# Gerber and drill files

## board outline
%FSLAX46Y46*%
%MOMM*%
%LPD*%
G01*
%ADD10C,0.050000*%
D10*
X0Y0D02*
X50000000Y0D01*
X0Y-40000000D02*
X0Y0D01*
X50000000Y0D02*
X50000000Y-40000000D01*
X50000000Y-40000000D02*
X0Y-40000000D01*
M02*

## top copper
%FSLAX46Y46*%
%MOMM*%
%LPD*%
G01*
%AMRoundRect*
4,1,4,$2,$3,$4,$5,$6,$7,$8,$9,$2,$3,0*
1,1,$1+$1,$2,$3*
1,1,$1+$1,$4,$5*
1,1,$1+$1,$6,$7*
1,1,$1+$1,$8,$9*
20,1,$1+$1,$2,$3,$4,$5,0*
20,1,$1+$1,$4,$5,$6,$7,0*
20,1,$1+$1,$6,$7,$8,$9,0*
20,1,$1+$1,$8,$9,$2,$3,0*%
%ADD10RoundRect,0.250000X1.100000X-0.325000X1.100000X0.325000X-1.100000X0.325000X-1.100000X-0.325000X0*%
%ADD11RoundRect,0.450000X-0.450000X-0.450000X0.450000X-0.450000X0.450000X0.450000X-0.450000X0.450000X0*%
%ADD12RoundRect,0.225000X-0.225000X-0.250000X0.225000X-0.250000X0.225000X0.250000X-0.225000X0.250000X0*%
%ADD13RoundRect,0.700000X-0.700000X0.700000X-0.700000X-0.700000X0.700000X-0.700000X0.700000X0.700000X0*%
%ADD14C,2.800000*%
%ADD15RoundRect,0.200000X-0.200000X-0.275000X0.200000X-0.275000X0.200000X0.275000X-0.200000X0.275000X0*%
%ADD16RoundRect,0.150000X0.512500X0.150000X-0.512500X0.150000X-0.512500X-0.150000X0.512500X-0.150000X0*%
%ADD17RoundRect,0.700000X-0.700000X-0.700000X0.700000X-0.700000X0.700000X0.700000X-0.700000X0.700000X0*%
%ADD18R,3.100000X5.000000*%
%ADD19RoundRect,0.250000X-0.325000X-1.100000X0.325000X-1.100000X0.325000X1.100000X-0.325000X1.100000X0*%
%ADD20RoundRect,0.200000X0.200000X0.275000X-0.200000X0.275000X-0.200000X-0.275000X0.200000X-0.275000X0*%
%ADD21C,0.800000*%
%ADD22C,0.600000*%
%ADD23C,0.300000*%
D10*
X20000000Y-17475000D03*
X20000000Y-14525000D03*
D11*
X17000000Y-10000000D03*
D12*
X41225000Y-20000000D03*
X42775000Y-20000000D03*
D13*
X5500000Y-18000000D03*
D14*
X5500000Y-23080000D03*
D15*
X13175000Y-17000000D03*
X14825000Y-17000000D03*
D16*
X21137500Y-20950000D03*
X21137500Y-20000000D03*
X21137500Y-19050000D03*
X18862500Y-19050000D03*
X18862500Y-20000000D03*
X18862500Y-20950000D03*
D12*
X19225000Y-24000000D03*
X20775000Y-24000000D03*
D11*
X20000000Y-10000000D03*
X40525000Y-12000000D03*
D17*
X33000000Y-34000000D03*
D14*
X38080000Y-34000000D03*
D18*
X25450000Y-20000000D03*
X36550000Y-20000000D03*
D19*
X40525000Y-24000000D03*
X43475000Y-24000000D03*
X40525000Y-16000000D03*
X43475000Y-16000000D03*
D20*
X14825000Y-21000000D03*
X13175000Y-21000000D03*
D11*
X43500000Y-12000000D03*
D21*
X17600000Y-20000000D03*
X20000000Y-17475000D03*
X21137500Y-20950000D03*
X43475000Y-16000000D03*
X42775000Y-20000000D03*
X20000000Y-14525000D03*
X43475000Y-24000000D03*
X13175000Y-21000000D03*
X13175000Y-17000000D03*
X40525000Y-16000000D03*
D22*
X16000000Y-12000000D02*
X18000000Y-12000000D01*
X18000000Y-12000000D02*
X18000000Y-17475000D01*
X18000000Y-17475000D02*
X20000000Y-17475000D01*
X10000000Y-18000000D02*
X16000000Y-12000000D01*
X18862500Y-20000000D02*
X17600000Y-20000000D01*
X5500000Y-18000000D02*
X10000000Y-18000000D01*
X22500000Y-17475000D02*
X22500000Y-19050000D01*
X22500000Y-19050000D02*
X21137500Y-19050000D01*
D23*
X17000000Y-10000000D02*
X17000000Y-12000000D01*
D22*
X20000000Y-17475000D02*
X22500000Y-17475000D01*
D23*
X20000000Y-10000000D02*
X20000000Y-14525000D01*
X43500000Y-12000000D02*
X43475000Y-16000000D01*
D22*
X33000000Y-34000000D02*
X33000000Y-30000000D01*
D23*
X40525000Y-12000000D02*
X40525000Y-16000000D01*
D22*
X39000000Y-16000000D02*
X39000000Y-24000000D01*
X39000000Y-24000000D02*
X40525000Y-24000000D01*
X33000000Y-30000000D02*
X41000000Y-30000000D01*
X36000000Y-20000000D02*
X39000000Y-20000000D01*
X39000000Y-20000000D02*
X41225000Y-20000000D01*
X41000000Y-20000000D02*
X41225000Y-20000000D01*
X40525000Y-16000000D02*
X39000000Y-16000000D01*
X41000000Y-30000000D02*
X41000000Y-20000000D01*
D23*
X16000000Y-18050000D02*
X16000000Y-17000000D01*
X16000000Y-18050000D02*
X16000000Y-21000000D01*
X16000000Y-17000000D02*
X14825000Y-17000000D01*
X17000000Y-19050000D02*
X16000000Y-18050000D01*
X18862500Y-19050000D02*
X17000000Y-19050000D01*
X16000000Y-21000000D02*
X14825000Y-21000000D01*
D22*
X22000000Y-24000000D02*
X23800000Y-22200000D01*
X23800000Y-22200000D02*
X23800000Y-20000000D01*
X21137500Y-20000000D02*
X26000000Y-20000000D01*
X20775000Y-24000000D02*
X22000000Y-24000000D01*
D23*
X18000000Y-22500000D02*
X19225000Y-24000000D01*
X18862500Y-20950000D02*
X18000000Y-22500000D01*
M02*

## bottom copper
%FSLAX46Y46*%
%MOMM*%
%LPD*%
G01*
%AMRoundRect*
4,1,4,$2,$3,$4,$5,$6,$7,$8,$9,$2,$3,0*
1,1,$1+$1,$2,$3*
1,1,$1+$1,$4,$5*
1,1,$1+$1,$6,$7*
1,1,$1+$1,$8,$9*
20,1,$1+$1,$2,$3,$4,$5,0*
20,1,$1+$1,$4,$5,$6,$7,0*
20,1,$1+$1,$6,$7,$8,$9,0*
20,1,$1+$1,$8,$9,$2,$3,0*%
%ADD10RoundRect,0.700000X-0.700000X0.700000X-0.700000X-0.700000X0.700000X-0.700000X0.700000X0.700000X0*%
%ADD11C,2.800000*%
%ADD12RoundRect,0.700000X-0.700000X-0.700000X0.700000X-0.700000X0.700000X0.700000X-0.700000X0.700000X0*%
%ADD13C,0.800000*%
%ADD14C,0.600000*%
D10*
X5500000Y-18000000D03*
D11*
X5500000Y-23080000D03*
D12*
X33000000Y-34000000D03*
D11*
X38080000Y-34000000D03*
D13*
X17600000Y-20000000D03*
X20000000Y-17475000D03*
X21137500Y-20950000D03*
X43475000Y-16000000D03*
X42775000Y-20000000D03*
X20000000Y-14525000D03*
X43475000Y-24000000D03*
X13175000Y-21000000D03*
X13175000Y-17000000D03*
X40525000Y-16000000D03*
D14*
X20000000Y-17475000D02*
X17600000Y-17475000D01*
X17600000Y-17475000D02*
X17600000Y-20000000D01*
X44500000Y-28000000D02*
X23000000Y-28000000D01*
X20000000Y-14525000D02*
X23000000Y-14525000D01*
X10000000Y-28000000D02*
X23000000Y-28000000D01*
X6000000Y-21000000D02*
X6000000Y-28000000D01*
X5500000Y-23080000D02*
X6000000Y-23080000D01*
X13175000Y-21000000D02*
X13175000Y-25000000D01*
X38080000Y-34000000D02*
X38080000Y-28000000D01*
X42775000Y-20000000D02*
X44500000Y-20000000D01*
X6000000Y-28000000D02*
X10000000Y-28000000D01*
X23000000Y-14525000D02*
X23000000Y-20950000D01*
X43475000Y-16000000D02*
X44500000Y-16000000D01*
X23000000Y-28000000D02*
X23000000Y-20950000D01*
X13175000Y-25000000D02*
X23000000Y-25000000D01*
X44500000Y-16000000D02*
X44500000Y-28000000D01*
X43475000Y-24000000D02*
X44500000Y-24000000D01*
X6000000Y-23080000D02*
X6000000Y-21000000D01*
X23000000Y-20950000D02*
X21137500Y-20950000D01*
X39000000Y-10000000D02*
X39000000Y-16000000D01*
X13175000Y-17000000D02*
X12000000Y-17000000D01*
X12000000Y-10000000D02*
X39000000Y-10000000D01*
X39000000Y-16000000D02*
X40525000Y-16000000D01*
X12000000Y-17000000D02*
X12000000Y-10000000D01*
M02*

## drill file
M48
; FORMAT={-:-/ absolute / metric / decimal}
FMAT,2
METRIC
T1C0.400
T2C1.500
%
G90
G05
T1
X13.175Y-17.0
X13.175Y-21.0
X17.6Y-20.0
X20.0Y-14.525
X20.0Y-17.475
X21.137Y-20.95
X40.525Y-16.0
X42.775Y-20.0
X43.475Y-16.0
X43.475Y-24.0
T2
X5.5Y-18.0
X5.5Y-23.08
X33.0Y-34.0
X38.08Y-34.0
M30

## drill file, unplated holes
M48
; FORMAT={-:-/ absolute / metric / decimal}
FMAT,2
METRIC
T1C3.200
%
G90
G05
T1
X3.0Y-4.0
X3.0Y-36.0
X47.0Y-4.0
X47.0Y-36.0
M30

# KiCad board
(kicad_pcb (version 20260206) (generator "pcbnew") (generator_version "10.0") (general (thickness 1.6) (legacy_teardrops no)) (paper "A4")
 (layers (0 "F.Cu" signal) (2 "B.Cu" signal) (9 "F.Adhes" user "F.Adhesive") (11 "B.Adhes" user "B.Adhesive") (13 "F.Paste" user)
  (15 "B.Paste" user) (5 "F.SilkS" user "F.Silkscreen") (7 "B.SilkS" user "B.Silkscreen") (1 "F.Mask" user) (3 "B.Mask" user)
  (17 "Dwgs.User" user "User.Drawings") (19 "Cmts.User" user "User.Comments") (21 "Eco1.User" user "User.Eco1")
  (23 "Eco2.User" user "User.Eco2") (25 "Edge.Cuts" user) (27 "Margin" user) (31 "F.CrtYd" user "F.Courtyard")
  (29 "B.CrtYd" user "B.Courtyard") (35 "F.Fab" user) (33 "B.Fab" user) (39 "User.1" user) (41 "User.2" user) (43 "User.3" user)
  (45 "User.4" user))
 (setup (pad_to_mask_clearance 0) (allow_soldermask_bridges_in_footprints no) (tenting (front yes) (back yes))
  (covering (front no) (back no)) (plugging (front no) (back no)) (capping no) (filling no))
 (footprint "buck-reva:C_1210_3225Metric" (layer "F.Cu") (at 20 16 90)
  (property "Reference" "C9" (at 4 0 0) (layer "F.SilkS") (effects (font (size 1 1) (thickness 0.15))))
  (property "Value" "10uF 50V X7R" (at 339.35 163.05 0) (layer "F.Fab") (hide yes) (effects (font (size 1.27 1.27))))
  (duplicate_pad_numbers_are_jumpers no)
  (pad "1" smd roundrect (at -1.475 0 90) (size 1.15 2.7) (layers "F.Cu" "F.Mask" "F.Paste") (roundrect_rratio 0.217391) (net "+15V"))
  (pad "2" smd roundrect (at 1.475 0 90) (size 1.15 2.7) (layers "F.Cu" "F.Mask" "F.Paste") (roundrect_rratio 0.217391) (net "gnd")))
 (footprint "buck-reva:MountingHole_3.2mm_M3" (layer "F.Cu") (at 3 36)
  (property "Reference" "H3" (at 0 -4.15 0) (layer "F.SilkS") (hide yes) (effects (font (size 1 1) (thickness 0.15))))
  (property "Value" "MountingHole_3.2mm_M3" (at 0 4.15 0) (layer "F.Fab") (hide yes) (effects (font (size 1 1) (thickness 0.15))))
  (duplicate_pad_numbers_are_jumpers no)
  (pad "" np_thru_hole circle (at 0 0) (size 3.2 3.2) (drill 3.2) (layers "*.Cu" "*.Mask")))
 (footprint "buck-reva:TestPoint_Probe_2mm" (layer "F.Cu") (at 17 10)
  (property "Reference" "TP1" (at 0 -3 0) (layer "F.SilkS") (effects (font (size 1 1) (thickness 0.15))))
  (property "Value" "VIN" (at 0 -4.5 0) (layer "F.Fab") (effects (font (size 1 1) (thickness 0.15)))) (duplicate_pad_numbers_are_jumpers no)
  (pad "1" smd roundrect (at 0 0) (size 1.8 1.8) (layers "F.Cu" "F.Mask") (roundrect_rratio 0.25) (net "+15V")))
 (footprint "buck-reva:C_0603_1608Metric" (layer "F.Cu") (at 42 20)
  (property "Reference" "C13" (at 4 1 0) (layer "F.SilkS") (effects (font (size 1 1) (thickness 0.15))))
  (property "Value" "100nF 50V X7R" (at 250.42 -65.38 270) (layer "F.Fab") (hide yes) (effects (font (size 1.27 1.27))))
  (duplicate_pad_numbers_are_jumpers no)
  (pad "1" smd roundrect (at -0.775 0) (size 0.9 0.95) (layers "F.Cu" "F.Mask" "F.Paste") (roundrect_rratio 0.25) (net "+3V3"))
  (pad "2" smd roundrect (at 0.775 0) (size 0.9 0.95) (layers "F.Cu" "F.Mask" "F.Paste") (roundrect_rratio 0.25) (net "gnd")))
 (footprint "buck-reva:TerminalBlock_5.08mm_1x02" (layer "F.Cu") (at 5.5 18 -90)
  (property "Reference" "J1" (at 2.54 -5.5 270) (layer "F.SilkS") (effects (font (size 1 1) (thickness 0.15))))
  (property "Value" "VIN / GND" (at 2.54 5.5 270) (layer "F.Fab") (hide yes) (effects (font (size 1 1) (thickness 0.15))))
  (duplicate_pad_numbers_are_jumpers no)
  (pad "1" thru_hole roundrect (at 0 0 270) (size 2.8 2.8) (drill 1.5) (layers "*.Cu" "*.Mask") (remove_unused_layers no)
   (roundrect_rratio 0.25) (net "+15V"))
  (pad "2" thru_hole circle (at 5.08 0 270) (size 2.8 2.8) (drill 1.5) (layers "*.Cu" "*.Mask") (remove_unused_layers no) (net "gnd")))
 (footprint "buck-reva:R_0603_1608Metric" (layer "F.Cu") (at 14 17)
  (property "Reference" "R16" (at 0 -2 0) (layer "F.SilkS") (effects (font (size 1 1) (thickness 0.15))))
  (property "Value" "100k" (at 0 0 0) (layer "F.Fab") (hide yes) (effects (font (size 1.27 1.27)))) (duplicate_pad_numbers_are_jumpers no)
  (pad "1" smd roundrect (at -0.825 0) (size 0.8 0.95) (layers "F.Cu" "F.Mask" "F.Paste") (roundrect_rratio 0.25) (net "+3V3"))
  (pad "2" smd roundrect (at 0.825 0) (size 0.8 0.95) (layers "F.Cu" "F.Mask" "F.Paste") (roundrect_rratio 0.25) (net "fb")))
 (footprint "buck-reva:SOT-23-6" (layer "F.Cu") (at 20 20 180)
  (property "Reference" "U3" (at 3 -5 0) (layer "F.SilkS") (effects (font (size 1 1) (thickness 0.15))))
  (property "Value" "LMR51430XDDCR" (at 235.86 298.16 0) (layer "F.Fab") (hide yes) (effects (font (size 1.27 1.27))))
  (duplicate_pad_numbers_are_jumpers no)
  (pad "1" smd roundrect (at -1.1375 -0.95 180) (size 1.325 0.6) (layers "F.Cu" "F.Mask" "F.Paste") (roundrect_rratio 0.25) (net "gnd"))
  (pad "2" smd roundrect (at -1.1375 0 180) (size 1.325 0.6) (layers "F.Cu" "F.Mask" "F.Paste") (roundrect_rratio 0.25) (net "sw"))
  (pad "3" smd roundrect (at -1.1375 0.95 180) (size 1.325 0.6) (layers "F.Cu" "F.Mask" "F.Paste") (roundrect_rratio 0.25) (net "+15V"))
  (pad "4" smd roundrect (at 1.1375 0.95 180) (size 1.325 0.6) (layers "F.Cu" "F.Mask" "F.Paste") (roundrect_rratio 0.25) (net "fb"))
  (pad "5" smd roundrect (at 1.1375 0 180) (size 1.325 0.6) (layers "F.Cu" "F.Mask" "F.Paste") (roundrect_rratio 0.25) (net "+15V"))
  (pad "6" smd roundrect (at 1.1375 -0.95 180) (size 1.325 0.6) (layers "F.Cu" "F.Mask" "F.Paste") (roundrect_rratio 0.25) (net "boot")))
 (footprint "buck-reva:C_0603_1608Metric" (layer "F.Cu") (at 20 24)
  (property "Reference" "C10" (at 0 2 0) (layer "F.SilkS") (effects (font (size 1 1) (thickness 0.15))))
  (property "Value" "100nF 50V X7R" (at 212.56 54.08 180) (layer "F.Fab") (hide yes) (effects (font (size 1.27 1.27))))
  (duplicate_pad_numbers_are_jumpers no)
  (pad "1" smd roundrect (at -0.775 0) (size 0.9 0.95) (layers "F.Cu" "F.Mask" "F.Paste") (roundrect_rratio 0.25) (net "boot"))
  (pad "2" smd roundrect (at 0.775 0) (size 0.9 0.95) (layers "F.Cu" "F.Mask" "F.Paste") (roundrect_rratio 0.25) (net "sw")))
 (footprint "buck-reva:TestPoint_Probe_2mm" (layer "F.Cu") (at 20 10)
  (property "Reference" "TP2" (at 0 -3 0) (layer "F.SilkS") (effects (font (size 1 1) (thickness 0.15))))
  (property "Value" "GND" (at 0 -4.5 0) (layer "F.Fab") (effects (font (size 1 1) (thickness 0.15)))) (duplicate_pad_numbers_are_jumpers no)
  (pad "1" smd roundrect (at 0 0) (size 1.8 1.8) (layers "F.Cu" "F.Mask") (roundrect_rratio 0.25) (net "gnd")))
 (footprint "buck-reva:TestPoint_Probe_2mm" (layer "F.Cu") (at 40.525 12)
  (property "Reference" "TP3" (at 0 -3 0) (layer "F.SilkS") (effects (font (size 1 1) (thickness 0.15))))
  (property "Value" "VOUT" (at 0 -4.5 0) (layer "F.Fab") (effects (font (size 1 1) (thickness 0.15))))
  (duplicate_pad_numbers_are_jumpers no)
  (pad "1" smd roundrect (at 0 0) (size 1.8 1.8) (layers "F.Cu" "F.Mask") (roundrect_rratio 0.25) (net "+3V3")))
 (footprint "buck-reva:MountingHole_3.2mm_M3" (layer "F.Cu") (at 47 4)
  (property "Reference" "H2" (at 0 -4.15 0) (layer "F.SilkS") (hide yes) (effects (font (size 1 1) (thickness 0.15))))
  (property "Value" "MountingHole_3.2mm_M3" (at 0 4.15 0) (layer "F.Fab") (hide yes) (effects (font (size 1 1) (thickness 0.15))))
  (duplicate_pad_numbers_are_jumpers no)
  (pad "" np_thru_hole circle (at 0 0) (size 3.2 3.2) (drill 3.2) (layers "*.Cu" "*.Mask")))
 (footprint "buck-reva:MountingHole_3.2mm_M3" (layer "F.Cu") (at 3 4)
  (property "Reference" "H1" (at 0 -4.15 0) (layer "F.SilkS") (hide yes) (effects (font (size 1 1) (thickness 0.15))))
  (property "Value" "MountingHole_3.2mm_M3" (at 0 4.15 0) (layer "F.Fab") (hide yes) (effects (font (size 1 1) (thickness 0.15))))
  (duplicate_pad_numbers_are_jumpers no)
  (pad "" np_thru_hole circle (at 0 0) (size 3.2 3.2) (drill 3.2) (layers "*.Cu" "*.Mask")))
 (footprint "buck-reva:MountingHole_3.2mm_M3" (layer "F.Cu") (at 47 36)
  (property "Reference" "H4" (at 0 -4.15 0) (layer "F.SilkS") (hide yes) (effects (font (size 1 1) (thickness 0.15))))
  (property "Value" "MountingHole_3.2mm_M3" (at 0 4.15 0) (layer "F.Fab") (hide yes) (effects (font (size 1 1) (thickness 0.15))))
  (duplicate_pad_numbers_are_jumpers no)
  (pad "" np_thru_hole circle (at 0 0) (size 3.2 3.2) (drill 3.2) (layers "*.Cu" "*.Mask")))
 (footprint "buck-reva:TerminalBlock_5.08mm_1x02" (layer "F.Cu") (at 33 34)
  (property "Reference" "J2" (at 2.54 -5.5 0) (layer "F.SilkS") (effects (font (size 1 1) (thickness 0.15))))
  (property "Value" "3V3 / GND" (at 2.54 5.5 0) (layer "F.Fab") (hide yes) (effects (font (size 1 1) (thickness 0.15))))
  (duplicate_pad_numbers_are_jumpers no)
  (pad "1" thru_hole roundrect (at 0 0) (size 2.8 2.8) (drill 1.5) (layers "*.Cu" "*.Mask") (remove_unused_layers no)
   (roundrect_rratio 0.25) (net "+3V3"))
  (pad "2" thru_hole circle (at 5.08 0) (size 2.8 2.8) (drill 1.5) (layers "*.Cu" "*.Mask") (remove_unused_layers no) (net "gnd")))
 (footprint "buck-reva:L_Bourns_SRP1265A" (layer "F.Cu") (at 31 20)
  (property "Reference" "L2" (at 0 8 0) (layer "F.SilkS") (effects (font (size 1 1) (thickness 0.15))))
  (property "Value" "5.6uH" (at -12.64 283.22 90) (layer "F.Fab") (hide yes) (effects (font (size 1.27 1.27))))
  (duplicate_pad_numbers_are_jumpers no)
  (pad "1" smd rect (at -5.55 0) (size 3.1 5) (layers "F.Cu" "F.Mask" "F.Paste") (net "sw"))
  (pad "2" smd rect (at 5.55 0) (size 3.1 5) (layers "F.Cu" "F.Mask" "F.Paste") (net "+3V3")))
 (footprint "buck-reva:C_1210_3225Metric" (layer "F.Cu") (at 42 24)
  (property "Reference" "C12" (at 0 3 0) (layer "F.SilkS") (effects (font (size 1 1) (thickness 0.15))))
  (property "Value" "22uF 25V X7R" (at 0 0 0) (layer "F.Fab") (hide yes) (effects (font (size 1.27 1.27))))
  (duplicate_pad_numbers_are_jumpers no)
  (pad "1" smd roundrect (at -1.475 0) (size 1.15 2.7) (layers "F.Cu" "F.Mask" "F.Paste") (roundrect_rratio 0.217391) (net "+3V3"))
  (pad "2" smd roundrect (at 1.475 0) (size 1.15 2.7) (layers "F.Cu" "F.Mask" "F.Paste") (roundrect_rratio 0.217391) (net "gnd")))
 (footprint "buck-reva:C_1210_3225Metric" (layer "F.Cu") (at 42 16)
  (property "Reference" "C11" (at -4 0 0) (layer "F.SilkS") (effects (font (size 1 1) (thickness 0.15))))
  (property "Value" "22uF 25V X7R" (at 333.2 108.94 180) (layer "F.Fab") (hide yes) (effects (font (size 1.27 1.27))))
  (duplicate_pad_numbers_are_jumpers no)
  (pad "1" smd roundrect (at -1.475 0) (size 1.15 2.7) (layers "F.Cu" "F.Mask" "F.Paste") (roundrect_rratio 0.217391) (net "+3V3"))
  (pad "2" smd roundrect (at 1.475 0) (size 1.15 2.7) (layers "F.Cu" "F.Mask" "F.Paste") (roundrect_rratio 0.217391) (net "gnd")))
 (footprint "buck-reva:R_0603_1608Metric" (layer "F.Cu") (at 14 21 180)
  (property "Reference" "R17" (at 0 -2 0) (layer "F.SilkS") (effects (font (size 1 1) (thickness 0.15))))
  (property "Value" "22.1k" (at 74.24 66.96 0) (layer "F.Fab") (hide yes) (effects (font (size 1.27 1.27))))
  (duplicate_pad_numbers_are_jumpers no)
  (pad "1" smd roundrect (at -0.825 0 180) (size 0.8 0.95) (layers "F.Cu" "F.Mask" "F.Paste") (roundrect_rratio 0.25) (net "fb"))
  (pad "2" smd roundrect (at 0.825 0 180) (size 0.8 0.95) (layers "F.Cu" "F.Mask" "F.Paste") (roundrect_rratio 0.25) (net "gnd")))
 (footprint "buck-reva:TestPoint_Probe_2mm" (layer "F.Cu") (at 43.5 12)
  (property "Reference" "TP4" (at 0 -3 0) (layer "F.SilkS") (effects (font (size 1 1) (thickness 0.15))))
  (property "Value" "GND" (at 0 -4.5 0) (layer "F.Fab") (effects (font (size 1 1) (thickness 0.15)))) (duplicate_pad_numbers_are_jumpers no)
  (pad "1" smd roundrect (at 0 0) (size 1.8 1.8) (layers "F.Cu" "F.Mask") (roundrect_rratio 0.25) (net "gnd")))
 (gr_line (start 0 0) (end 50 0) (stroke (width 0.05) (type default)) (layer "Edge.Cuts"))
 (gr_line (start 0 40) (end 0 0) (stroke (width 0.05) (type default)) (layer "Edge.Cuts"))
 (gr_line (start 50 0) (end 50 40) (stroke (width 0.05) (type default)) (layer "Edge.Cuts"))
 (gr_line (start 50 40) (end 0 40) (stroke (width 0.05) (type default)) (layer "Edge.Cuts"))
 (segment (start 16 12) (end 18 12) (width 0.6) (layer "F.Cu") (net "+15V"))
 (segment (start 18 12) (end 18 17.475) (width 0.6) (layer "F.Cu") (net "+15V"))
 (segment (start 18 17.475) (end 20 17.475) (width 0.6) (layer "F.Cu") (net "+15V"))
 (segment (start 10 18) (end 16 12) (width 0.6) (layer "F.Cu") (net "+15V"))
 (segment (start 18.8625 20) (end 17.6 20) (width 0.6) (layer "F.Cu") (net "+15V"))
 (segment (start 5.5 18) (end 10 18) (width 0.6) (layer "F.Cu") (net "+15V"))
 (segment (start 22.5 17.475) (end 22.5 19.05) (width 0.6) (layer "F.Cu") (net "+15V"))
 (segment (start 22.5 19.05) (end 21.1375 19.05) (width 0.6) (layer "F.Cu") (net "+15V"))
 (segment (start 17 10) (end 17 12) (width 0.3) (layer "F.Cu") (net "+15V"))
 (segment (start 20 17.475) (end 22.5 17.475) (width 0.6) (layer "F.Cu") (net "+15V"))
 (via (at 17.6 20) (size 0.8) (drill 0.4) (layers "F.Cu" "B.Cu") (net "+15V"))
 (via (at 20 17.475) (size 0.8) (drill 0.4) (layers "F.Cu" "B.Cu") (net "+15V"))
 (segment (start 20 17.475) (end 17.6 17.475) (width 0.6) (layer "B.Cu") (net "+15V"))
 (segment (start 17.6 17.475) (end 17.6 20) (width 0.6) (layer "B.Cu") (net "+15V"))
 (segment (start 20 10) (end 20 14.525) (width 0.3) (layer "F.Cu") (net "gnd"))
 (segment (start 43.5 12) (end 43.475 16) (width 0.3) (layer "F.Cu") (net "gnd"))
 (via (at 21.1375 20.95) (size 0.8) (drill 0.4) (layers "F.Cu" "B.Cu") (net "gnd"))
 (via (at 43.475 16) (size 0.8) (drill 0.4) (layers "F.Cu" "B.Cu") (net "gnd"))
 (via (at 42.775 20) (size 0.8) (drill 0.4) (layers "F.Cu" "B.Cu") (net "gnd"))
 (via (at 20 14.525) (size 0.8) (drill 0.4) (layers "F.Cu" "B.Cu") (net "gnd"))
 (via (at 43.475 24) (size 0.8) (drill 0.4) (layers "F.Cu" "B.Cu") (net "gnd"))
 (via (at 13.175 21) (size 0.8) (drill 0.4) (layers "F.Cu" "B.Cu") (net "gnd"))
 (segment (start 44.5 28) (end 23 28) (width 0.6) (layer "B.Cu") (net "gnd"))
 (segment (start 20 14.525) (end 23 14.525) (width 0.6) (layer "B.Cu") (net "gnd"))
 (segment (start 10 28) (end 23 28) (width 0.6) (layer "B.Cu") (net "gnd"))
 (segment (start 6 21) (end 6 28) (width 0.6) (layer "B.Cu") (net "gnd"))
 (segment (start 5.5 23.08) (end 6 23.08) (width 0.6) (layer "B.Cu") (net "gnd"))
 (segment (start 13.175 21) (end 13.175 25) (width 0.6) (layer "B.Cu") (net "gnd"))
 (segment (start 38.08 34) (end 38.08 28) (width 0.6) (layer "B.Cu") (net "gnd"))
 (segment (start 42.775 20) (end 44.5 20) (width 0.6) (layer "B.Cu") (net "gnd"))
 (segment (start 6 28) (end 10 28) (width 0.6) (layer "B.Cu") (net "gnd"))
 (segment (start 23 14.525) (end 23 20.95) (width 0.6) (layer "B.Cu") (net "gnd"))
 (segment (start 43.475 16) (end 44.5 16) (width 0.6) (layer "B.Cu") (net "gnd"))
 (segment (start 23 28) (end 23 20.95) (width 0.6) (layer "B.Cu") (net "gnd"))
 (segment (start 13.175 25) (end 23 25) (width 0.6) (layer "B.Cu") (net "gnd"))
 (segment (start 44.5 16) (end 44.5 28) (width 0.6) (layer "B.Cu") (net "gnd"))
 (segment (start 43.475 24) (end 44.5 24) (width 0.6) (layer "B.Cu") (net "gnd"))
 (segment (start 6 23.08) (end 6 21) (width 0.6) (layer "B.Cu") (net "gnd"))
 (segment (start 23 20.95) (end 21.1375 20.95) (width 0.6) (layer "B.Cu") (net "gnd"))
 (segment (start 33 34) (end 33 30) (width 0.6) (layer "F.Cu") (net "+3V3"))
 (segment (start 40.525 12) (end 40.525 16) (width 0.3) (layer "F.Cu") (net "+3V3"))
 (segment (start 39 16) (end 39 24) (width 0.6) (layer "F.Cu") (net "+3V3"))
 (segment (start 39 24) (end 40.525 24) (width 0.6) (layer "F.Cu") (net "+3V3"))
 (segment (start 33 30) (end 41 30) (width 0.6) (layer "F.Cu") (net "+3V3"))
 (segment (start 36 20) (end 39 20) (width 0.6) (layer "F.Cu") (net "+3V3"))
 (segment (start 39 20) (end 41.225 20) (width 0.6) (layer "F.Cu") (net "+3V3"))
 (segment (start 41 20) (end 41.225 20) (width 0.6) (layer "F.Cu") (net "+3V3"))
 (segment (start 40.525 16) (end 39 16) (width 0.6) (layer "F.Cu") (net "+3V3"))
 (segment (start 41 30) (end 41 20) (width 0.6) (layer "F.Cu") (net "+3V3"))
 (via (at 13.175 17) (size 0.8) (drill 0.4) (layers "F.Cu" "B.Cu") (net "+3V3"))
 (via (at 40.525 16) (size 0.8) (drill 0.4) (layers "F.Cu" "B.Cu") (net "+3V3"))
 (segment (start 39 10) (end 39 16) (width 0.6) (layer "B.Cu") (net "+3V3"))
 (segment (start 13.175 17) (end 12 17) (width 0.6) (layer "B.Cu") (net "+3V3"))
 (segment (start 12 10) (end 39 10) (width 0.6) (layer "B.Cu") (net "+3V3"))
 (segment (start 39 16) (end 40.525 16) (width 0.6) (layer "B.Cu") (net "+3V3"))
 (segment (start 12 17) (end 12 10) (width 0.6) (layer "B.Cu") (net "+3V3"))
 (segment (start 16 18.05) (end 16 17) (width 0.3) (layer "F.Cu") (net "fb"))
 (segment (start 16 18.05) (end 16 21) (width 0.3) (layer "F.Cu") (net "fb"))
 (segment (start 16 17) (end 14.825 17) (width 0.3) (layer "F.Cu") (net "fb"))
 (segment (start 17 19.05) (end 16 18.05) (width 0.3) (layer "F.Cu") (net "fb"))
 (segment (start 18.8625 19.05) (end 17 19.05) (width 0.3) (layer "F.Cu") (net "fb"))
 (segment (start 16 21) (end 14.825 21) (width 0.3) (layer "F.Cu") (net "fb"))
 (segment (start 22 24) (end 23.8 22.2) (width 0.6) (layer "F.Cu") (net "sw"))
 (segment (start 23.8 22.2) (end 23.8 20) (width 0.6) (layer "F.Cu") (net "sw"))
 (segment (start 21.1375 20) (end 26 20) (width 0.6) (layer "F.Cu") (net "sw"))
 (segment (start 20.775 24) (end 22 24) (width 0.6) (layer "F.Cu") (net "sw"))
 (segment (start 18 22.5) (end 19.225 24) (width 0.3) (layer "F.Cu") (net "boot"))
 (segment (start 18.8625 20.95) (end 18 22.5) (width 0.3) (layer "F.Cu") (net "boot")))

